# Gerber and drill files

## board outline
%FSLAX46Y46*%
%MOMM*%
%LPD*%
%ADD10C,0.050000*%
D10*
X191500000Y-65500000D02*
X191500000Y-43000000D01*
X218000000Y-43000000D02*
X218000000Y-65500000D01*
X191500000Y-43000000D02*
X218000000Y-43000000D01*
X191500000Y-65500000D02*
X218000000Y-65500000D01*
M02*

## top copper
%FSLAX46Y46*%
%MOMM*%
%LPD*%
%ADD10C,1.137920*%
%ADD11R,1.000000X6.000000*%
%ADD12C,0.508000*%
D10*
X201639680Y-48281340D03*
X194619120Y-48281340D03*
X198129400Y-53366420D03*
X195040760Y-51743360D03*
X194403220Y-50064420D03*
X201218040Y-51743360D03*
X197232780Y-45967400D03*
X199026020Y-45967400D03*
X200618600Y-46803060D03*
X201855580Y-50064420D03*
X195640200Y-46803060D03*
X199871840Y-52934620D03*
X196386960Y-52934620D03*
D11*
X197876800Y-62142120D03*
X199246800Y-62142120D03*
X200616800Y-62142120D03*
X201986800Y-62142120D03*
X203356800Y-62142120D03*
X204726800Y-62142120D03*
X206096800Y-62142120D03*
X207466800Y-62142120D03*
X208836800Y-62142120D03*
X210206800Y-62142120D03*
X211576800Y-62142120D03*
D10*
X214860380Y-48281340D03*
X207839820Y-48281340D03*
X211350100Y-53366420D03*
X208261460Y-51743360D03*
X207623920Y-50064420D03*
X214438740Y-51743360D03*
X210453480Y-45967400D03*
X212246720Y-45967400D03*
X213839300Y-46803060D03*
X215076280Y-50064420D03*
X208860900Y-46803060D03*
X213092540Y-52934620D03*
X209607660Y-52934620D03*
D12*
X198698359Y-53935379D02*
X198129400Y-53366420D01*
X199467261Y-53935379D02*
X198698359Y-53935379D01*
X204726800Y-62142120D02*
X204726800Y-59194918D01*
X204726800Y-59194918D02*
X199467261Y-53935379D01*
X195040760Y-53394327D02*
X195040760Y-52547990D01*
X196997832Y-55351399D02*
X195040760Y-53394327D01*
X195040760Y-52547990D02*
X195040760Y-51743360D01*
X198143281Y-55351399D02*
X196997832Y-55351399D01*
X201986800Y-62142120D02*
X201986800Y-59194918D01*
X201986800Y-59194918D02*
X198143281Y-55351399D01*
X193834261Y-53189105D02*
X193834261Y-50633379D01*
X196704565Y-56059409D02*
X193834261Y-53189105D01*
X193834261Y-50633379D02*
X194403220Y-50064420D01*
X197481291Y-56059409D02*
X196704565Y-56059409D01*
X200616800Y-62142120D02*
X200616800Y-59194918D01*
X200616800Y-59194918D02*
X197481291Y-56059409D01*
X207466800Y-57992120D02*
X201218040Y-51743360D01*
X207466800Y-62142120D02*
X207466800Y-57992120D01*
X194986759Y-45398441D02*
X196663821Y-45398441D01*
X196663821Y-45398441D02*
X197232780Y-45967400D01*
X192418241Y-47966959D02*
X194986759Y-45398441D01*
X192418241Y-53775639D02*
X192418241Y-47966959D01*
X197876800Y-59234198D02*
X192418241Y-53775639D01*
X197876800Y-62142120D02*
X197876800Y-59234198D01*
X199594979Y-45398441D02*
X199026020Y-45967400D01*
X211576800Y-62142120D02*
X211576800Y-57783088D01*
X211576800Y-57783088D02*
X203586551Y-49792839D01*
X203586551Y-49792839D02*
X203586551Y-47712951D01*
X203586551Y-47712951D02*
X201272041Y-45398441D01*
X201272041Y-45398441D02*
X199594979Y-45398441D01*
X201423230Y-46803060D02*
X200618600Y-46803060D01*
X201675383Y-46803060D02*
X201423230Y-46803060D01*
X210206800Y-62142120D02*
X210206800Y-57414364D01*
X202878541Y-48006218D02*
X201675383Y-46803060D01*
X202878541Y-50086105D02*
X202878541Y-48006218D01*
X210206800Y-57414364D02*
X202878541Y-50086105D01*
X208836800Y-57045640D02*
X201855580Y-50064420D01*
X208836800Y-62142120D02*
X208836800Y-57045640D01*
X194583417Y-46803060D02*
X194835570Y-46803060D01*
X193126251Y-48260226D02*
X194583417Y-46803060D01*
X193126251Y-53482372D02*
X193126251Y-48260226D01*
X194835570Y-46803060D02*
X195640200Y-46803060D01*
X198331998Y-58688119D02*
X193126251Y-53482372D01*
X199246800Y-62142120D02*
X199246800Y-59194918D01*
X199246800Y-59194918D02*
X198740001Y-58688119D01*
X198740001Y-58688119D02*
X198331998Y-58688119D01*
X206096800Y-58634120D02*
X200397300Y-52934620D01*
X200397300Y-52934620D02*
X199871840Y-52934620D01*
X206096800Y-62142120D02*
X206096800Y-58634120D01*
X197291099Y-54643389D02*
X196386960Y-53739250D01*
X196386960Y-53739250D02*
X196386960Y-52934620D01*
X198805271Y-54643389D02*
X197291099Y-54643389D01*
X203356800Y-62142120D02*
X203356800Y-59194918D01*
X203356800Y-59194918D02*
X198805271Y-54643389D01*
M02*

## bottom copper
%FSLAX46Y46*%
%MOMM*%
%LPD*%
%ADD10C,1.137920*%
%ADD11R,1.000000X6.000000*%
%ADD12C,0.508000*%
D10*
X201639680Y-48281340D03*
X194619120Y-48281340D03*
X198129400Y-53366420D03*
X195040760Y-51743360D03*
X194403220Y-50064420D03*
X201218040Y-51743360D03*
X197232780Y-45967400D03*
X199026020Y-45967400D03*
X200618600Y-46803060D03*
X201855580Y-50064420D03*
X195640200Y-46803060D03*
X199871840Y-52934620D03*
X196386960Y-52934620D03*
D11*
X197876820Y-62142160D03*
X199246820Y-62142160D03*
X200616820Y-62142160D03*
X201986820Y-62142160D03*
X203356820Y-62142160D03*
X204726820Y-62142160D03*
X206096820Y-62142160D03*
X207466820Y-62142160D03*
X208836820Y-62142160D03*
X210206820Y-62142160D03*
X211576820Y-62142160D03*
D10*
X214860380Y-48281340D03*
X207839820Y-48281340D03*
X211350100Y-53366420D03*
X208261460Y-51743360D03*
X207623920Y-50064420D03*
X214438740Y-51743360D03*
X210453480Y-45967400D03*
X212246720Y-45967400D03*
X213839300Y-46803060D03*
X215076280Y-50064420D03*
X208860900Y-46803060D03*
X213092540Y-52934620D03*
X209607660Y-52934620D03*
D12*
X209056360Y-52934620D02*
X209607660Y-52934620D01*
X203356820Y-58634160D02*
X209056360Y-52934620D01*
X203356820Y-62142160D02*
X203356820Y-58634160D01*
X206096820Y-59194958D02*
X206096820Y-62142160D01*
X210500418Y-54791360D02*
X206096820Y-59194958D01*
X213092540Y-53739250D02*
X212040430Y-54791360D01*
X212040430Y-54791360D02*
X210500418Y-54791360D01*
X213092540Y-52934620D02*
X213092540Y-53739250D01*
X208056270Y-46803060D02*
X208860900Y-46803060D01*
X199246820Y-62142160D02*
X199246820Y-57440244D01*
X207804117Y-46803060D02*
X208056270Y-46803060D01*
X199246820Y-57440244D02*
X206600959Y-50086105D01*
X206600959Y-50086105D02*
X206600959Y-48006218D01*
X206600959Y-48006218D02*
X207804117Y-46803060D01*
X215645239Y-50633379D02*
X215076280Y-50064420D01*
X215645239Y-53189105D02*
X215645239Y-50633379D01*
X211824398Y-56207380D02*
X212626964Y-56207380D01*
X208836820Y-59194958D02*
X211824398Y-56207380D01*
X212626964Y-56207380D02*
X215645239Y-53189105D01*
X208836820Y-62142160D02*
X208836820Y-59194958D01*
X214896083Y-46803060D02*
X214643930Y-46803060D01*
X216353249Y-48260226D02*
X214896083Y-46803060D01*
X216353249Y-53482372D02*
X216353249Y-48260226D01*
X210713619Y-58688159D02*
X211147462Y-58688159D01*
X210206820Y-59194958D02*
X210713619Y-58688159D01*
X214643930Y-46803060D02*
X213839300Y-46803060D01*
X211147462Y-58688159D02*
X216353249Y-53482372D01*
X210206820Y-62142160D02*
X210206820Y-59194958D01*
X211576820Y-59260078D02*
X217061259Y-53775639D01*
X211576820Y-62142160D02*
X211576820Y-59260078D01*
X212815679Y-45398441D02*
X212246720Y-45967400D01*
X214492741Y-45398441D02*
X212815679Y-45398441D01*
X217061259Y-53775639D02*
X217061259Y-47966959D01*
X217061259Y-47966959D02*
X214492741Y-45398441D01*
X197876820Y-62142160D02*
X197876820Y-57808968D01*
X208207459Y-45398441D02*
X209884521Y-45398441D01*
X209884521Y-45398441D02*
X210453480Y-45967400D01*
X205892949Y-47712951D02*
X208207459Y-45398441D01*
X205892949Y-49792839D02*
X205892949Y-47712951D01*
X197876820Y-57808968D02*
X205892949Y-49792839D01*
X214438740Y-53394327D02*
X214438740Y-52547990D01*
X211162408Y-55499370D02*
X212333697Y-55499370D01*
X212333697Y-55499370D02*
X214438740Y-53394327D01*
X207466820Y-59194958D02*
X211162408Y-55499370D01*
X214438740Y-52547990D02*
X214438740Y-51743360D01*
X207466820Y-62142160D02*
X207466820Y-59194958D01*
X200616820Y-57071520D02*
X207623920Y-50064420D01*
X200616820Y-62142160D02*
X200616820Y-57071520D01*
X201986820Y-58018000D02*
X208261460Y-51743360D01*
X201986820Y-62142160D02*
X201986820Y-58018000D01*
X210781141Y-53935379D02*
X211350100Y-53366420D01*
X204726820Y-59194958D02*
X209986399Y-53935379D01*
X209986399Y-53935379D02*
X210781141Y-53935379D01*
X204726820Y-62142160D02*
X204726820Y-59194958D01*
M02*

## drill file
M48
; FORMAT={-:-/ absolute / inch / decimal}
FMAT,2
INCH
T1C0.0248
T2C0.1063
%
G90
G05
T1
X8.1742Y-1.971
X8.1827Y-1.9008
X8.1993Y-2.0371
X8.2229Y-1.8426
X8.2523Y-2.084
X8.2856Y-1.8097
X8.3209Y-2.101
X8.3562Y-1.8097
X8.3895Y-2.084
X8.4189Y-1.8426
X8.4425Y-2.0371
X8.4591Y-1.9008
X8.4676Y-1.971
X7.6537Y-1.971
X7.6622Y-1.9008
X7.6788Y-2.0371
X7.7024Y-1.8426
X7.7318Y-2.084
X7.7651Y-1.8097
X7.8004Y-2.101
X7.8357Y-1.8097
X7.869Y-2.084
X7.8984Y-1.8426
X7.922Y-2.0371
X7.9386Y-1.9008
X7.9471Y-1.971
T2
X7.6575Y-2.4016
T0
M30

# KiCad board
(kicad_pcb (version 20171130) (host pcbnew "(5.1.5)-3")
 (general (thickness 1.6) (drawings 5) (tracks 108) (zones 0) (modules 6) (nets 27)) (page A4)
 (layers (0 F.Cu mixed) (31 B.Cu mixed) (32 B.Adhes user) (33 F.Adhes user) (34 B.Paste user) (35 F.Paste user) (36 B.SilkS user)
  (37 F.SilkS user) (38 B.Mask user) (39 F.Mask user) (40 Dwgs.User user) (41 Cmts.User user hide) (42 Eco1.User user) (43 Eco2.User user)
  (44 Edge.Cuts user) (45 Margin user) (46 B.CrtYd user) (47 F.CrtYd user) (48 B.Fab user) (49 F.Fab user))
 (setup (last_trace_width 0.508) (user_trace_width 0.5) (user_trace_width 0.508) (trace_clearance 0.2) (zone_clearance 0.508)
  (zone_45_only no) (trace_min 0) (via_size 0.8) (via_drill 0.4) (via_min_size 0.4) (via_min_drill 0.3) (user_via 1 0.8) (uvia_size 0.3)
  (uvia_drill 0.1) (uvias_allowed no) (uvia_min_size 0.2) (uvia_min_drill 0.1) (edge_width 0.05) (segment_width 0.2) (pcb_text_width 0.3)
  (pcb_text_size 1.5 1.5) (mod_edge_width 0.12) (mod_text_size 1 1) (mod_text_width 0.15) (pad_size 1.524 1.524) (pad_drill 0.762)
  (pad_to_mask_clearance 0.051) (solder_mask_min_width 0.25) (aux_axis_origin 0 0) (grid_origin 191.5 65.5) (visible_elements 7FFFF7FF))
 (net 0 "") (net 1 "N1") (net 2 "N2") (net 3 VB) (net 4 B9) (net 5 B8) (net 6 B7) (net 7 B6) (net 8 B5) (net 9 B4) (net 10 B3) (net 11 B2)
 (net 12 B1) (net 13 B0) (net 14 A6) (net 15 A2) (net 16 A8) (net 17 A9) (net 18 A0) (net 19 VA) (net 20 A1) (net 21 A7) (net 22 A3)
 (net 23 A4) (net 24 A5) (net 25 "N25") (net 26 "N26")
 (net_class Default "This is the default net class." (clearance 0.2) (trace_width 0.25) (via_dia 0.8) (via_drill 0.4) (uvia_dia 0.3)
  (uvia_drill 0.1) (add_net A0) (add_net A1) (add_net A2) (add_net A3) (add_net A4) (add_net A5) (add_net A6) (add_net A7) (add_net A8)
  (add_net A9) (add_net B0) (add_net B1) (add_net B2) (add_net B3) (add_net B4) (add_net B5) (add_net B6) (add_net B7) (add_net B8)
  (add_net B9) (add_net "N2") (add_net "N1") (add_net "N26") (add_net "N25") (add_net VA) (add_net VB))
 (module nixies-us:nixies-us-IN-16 (layer F.Cu) (at 198.1294 49.6123)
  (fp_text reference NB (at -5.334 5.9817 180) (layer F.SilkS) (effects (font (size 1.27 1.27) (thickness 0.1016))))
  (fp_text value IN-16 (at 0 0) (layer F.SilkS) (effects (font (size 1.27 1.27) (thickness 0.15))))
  (pad RHDP thru_hole circle (at 3.51028 -1.33096) (size 1.13792 1.13792) (drill 0.62992) (layers *.Cu *.Mask) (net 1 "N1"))
  (pad LHDP thru_hole circle (at -3.51028 -1.33096) (size 1.13792 1.13792) (drill 0.62992) (layers *.Cu *.Mask) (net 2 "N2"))
  (pad A thru_hole circle (at 0 3.75412) (size 1.13792 1.13792) (drill 0.62992) (layers *.Cu *.Mask) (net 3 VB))
  (pad 9 thru_hole circle (at -3.08864 2.13106) (size 1.13792 1.13792) (drill 0.62992) (layers *.Cu *.Mask) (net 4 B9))
  (pad 8 thru_hole circle (at -3.72618 0.45212) (size 1.13792 1.13792) (drill 0.62992) (layers *.Cu *.Mask) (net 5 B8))
  (pad 7 thru_hole circle (at 3.08864 2.13106) (size 1.13792 1.13792) (drill 0.62992) (layers *.Cu *.Mask) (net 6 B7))
  (pad 6 thru_hole circle (at -0.89662 -3.6449) (size 1.13792 1.13792) (drill 0.62992) (layers *.Cu *.Mask) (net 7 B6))
  (pad 5 thru_hole circle (at 0.89662 -3.6449) (size 1.13792 1.13792) (drill 0.62992) (layers *.Cu *.Mask) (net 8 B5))
  (pad 4 thru_hole circle (at 2.4892 -2.80924) (size 1.13792 1.13792) (drill 0.62992) (layers *.Cu *.Mask) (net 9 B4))
  (pad 3 thru_hole circle (at 3.72618 0.45212) (size 1.13792 1.13792) (drill 0.62992) (layers *.Cu *.Mask) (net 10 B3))
  (pad 2 thru_hole circle (at -2.4892 -2.80924) (size 1.13792 1.13792) (drill 0.62992) (layers *.Cu *.Mask) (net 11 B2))
  (pad 1 thru_hole circle (at 1.74244 3.32232) (size 1.13792 1.13792) (drill 0.62992) (layers *.Cu *.Mask) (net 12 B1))
  (pad 0 thru_hole circle (at -1.74244 3.32232) (size 1.13792 1.13792) (drill 0.62992) (layers *.Cu *.Mask) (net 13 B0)))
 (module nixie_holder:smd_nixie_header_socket (layer B.Cu) (at 197.87682 62.14216)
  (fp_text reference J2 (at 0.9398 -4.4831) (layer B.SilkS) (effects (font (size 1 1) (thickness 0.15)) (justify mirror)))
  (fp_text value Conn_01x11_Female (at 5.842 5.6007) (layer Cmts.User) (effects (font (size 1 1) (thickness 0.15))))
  (pad 1 smd rect (at 0 0) (size 1 6) (layers B.Cu B.Paste B.Mask) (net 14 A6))
  (pad 2 smd rect (at 1.37 0) (size 1 6) (layers B.Cu B.Paste B.Mask) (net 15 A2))
  (pad 3 smd rect (at 2.74 0) (size 1 6) (layers B.Cu B.Paste B.Mask) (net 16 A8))
  (pad 4 smd rect (at 4.11 0) (size 1 6) (layers B.Cu B.Paste B.Mask) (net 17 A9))
  (pad 5 smd rect (at 5.48 0) (size 1 6) (layers B.Cu B.Paste B.Mask) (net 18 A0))
  (pad 6 smd rect (at 6.85 0) (size 1 6) (layers B.Cu B.Paste B.Mask) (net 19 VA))
  (pad 7 smd rect (at 8.22 0) (size 1 6) (layers B.Cu B.Paste B.Mask) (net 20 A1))
  (pad 8 smd rect (at 9.59 0) (size 1 6) (layers B.Cu B.Paste B.Mask) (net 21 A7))
  (pad 9 smd rect (at 10.96 0) (size 1 6) (layers B.Cu B.Paste B.Mask) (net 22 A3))
  (pad 10 smd rect (at 12.33 0) (size 1 6) (layers B.Cu B.Paste B.Mask) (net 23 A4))
  (pad 11 smd rect (at 13.7 0) (size 1 6) (layers B.Cu B.Paste B.Mask) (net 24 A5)))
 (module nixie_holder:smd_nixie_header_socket (layer F.Cu) (at 197.8768 62.14212)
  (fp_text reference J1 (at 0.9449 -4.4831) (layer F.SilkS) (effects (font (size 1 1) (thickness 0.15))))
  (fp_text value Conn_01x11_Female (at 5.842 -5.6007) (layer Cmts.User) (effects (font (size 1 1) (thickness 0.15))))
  (pad 1 smd rect (at 0 0) (size 1 6) (layers F.Cu F.Paste F.Mask) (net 7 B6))
  (pad 2 smd rect (at 1.37 0) (size 1 6) (layers F.Cu F.Paste F.Mask) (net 11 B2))
  (pad 3 smd rect (at 2.74 0) (size 1 6) (layers F.Cu F.Paste F.Mask) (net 5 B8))
  (pad 4 smd rect (at 4.11 0) (size 1 6) (layers F.Cu F.Paste F.Mask) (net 4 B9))
  (pad 5 smd rect (at 5.48 0) (size 1 6) (layers F.Cu F.Paste F.Mask) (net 13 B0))
  (pad 6 smd rect (at 6.85 0) (size 1 6) (layers F.Cu F.Paste F.Mask) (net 3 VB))
  (pad 7 smd rect (at 8.22 0) (size 1 6) (layers F.Cu F.Paste F.Mask) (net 12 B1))
  (pad 8 smd rect (at 9.59 0) (size 1 6) (layers F.Cu F.Paste F.Mask) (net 6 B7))
  (pad 9 smd rect (at 10.96 0) (size 1 6) (layers F.Cu F.Paste F.Mask) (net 10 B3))
  (pad 10 smd rect (at 12.33 0) (size 1 6) (layers F.Cu F.Paste F.Mask) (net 9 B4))
  (pad 11 smd rect (at 13.7 0) (size 1 6) (layers F.Cu F.Paste F.Mask) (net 8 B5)))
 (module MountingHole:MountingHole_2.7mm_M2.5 (layer F.Cu) (at 194.5 61)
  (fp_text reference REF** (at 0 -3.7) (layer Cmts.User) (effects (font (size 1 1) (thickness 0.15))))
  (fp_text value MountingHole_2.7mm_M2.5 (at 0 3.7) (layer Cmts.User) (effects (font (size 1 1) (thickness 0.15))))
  (pad 1 np_thru_hole circle (at 0 0) (size 2.7 2.7) (drill 2.7) (layers *.Cu *.Mask)))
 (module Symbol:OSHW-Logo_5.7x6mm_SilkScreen (layer F.Cu) (at 204.708 55.81244)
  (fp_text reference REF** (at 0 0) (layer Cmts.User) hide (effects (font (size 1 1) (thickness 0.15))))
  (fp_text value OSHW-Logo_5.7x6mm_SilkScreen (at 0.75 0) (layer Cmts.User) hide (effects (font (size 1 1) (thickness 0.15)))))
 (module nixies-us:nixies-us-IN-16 (layer F.Cu) (at 211.3501 49.6123)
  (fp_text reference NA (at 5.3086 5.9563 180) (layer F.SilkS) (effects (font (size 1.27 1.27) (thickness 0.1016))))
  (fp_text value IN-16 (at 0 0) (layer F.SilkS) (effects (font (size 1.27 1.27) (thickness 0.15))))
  (pad RHDP thru_hole circle (at 3.51028 -1.33096) (size 1.13792 1.13792) (drill 0.62992) (layers *.Cu *.Mask) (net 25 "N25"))
  (pad LHDP thru_hole circle (at -3.51028 -1.33096) (size 1.13792 1.13792) (drill 0.62992) (layers *.Cu *.Mask) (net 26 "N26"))
  (pad A thru_hole circle (at 0 3.75412) (size 1.13792 1.13792) (drill 0.62992) (layers *.Cu *.Mask) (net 19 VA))
  (pad 9 thru_hole circle (at -3.08864 2.13106) (size 1.13792 1.13792) (drill 0.62992) (layers *.Cu *.Mask) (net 17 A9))
  (pad 8 thru_hole circle (at -3.72618 0.45212) (size 1.13792 1.13792) (drill 0.62992) (layers *.Cu *.Mask) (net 16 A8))
  (pad 7 thru_hole circle (at 3.08864 2.13106) (size 1.13792 1.13792) (drill 0.62992) (layers *.Cu *.Mask) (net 21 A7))
  (pad 6 thru_hole circle (at -0.89662 -3.6449) (size 1.13792 1.13792) (drill 0.62992) (layers *.Cu *.Mask) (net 14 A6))
  (pad 5 thru_hole circle (at 0.89662 -3.6449) (size 1.13792 1.13792) (drill 0.62992) (layers *.Cu *.Mask) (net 24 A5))
  (pad 4 thru_hole circle (at 2.4892 -2.80924) (size 1.13792 1.13792) (drill 0.62992) (layers *.Cu *.Mask) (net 23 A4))
  (pad 3 thru_hole circle (at 3.72618 0.45212) (size 1.13792 1.13792) (drill 0.62992) (layers *.Cu *.Mask) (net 22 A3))
  (pad 2 thru_hole circle (at -2.4892 -2.80924) (size 1.13792 1.13792) (drill 0.62992) (layers *.Cu *.Mask) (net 15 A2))
  (pad 1 thru_hole circle (at 1.74244 3.32232) (size 1.13792 1.13792) (drill 0.62992) (layers *.Cu *.Mask) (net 20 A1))
  (pad 0 thru_hole circle (at -1.74244 3.32232) (size 1.13792 1.13792) (drill 0.62992) (layers *.Cu *.Mask) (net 18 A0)))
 (gr_line (start 191.5 65.5) (end 191.5 43) (layer Edge.Cuts) (width 0.05))
 (gr_line (start 218 43) (end 218 65.5) (layer Edge.Cuts) (width 0.05))
 (gr_line (start 191.5 43) (end 218 43) (layer Edge.Cuts) (width 0.05))
 (gr_line (start 191.5 65.5) (end 218 65.5) (layer Edge.Cuts) (width 0.05))
 (segment (start 198.698359 53.935379) (end 198.1294 53.36642) (width 0.508) (layer F.Cu) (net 3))
 (segment (start 199.467261 53.935379) (end 198.698359 53.935379) (width 0.508) (layer F.Cu) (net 3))
 (segment (start 204.7268 62.14212) (end 204.7268 59.194918) (width 0.508) (layer F.Cu) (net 3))
 (segment (start 204.7268 59.194918) (end 199.467261 53.935379) (width 0.508) (layer F.Cu) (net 3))
 (segment (start 195.04076 53.394327) (end 195.04076 52.54799) (width 0.508) (layer F.Cu) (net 4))
 (segment (start 196.997832 55.351399) (end 195.04076 53.394327) (width 0.508) (layer F.Cu) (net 4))
 (segment (start 195.04076 52.54799) (end 195.04076 51.74336) (width 0.508) (layer F.Cu) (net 4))
 (segment (start 198.143281 55.351399) (end 196.997832 55.351399) (width 0.508) (layer F.Cu) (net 4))
 (segment (start 201.9868 62.14212) (end 201.9868 59.194918) (width 0.508) (layer F.Cu) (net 4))
 (segment (start 201.9868 59.194918) (end 198.143281 55.351399) (width 0.508) (layer F.Cu) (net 4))
 (segment (start 193.834261 53.189105) (end 193.834261 50.633379) (width 0.508) (layer F.Cu) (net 5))
 (segment (start 196.704565 56.059409) (end 193.834261 53.189105) (width 0.508) (layer F.Cu) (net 5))
 (segment (start 193.834261 50.633379) (end 194.40322 50.06442) (width 0.508) (layer F.Cu) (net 5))
 (segment (start 197.481291 56.059409) (end 196.704565 56.059409) (width 0.508) (layer F.Cu) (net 5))
 (segment (start 200.6168 62.14212) (end 200.6168 59.194918) (width 0.508) (layer F.Cu) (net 5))
 (segment (start 200.6168 59.194918) (end 197.481291 56.059409) (width 0.508) (layer F.Cu) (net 5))
 (segment (start 207.4668 57.99212) (end 201.21804 51.74336) (width 0.508) (layer F.Cu) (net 6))
 (segment (start 207.4668 62.14212) (end 207.4668 57.99212) (width 0.508) (layer F.Cu) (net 6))
 (segment (start 194.986759 45.398441) (end 196.663821 45.398441) (width 0.508) (layer F.Cu) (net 7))
 (segment (start 196.663821 45.398441) (end 197.23278 45.9674) (width 0.508) (layer F.Cu) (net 7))
 (segment (start 192.418241 47.966959) (end 194.986759 45.398441) (width 0.508) (layer F.Cu) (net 7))
 (segment (start 192.418241 53.775639) (end 192.418241 47.966959) (width 0.508) (layer F.Cu) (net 7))
 (segment (start 197.8768 59.234198) (end 192.418241 53.775639) (width 0.508) (layer F.Cu) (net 7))
 (segment (start 197.8768 62.14212) (end 197.8768 59.234198) (width 0.508) (layer F.Cu) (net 7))
 (segment (start 199.594979 45.398441) (end 199.02602 45.9674) (width 0.508) (layer F.Cu) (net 8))
 (segment (start 211.5768 62.14212) (end 211.5768 57.783088) (width 0.508) (layer F.Cu) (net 8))
 (segment (start 211.5768 57.783088) (end 203.586551 49.792839) (width 0.508) (layer F.Cu) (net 8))
 (segment (start 203.586551 49.792839) (end 203.586551 47.712951) (width 0.508) (layer F.Cu) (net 8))
 (segment (start 203.586551 47.712951) (end 201.272041 45.398441) (width 0.508) (layer F.Cu) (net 8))
 (segment (start 201.272041 45.398441) (end 199.594979 45.398441) (width 0.508) (layer F.Cu) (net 8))
 (segment (start 201.42323 46.80306) (end 200.6186 46.80306) (width 0.508) (layer F.Cu) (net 9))
 (segment (start 201.675383 46.80306) (end 201.42323 46.80306) (width 0.508) (layer F.Cu) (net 9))
 (segment (start 210.2068 62.14212) (end 210.2068 57.414364) (width 0.508) (layer F.Cu) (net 9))
 (segment (start 202.878541 48.006218) (end 201.675383 46.80306) (width 0.508) (layer F.Cu) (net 9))
 (segment (start 202.878541 50.086105) (end 202.878541 48.006218) (width 0.508) (layer F.Cu) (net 9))
 (segment (start 210.2068 57.414364) (end 202.878541 50.086105) (width 0.508) (layer F.Cu) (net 9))
 (segment (start 208.8368 57.04564) (end 201.85558 50.06442) (width 0.508) (layer F.Cu) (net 10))
 (segment (start 208.8368 62.14212) (end 208.8368 57.04564) (width 0.508) (layer F.Cu) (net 10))
 (segment (start 194.583417 46.80306) (end 194.83557 46.80306) (width 0.508) (layer F.Cu) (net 11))
 (segment (start 193.126251 48.260226) (end 194.583417 46.80306) (width 0.508) (layer F.Cu) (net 11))
 (segment (start 193.126251 53.482372) (end 193.126251 48.260226) (width 0.508) (layer F.Cu) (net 11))
 (segment (start 194.83557 46.80306) (end 195.6402 46.80306) (width 0.508) (layer F.Cu) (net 11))
 (segment (start 198.331998 58.688119) (end 193.126251 53.482372) (width 0.508) (layer F.Cu) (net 11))
 (segment (start 199.2468 62.14212) (end 199.2468 59.194918) (width 0.508) (layer F.Cu) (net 11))
 (segment (start 199.2468 59.194918) (end 198.740001 58.688119) (width 0.508) (layer F.Cu) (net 11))
 (segment (start 198.740001 58.688119) (end 198.331998 58.688119) (width 0.508) (layer F.Cu) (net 11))
 (segment (start 206.0968 58.63412) (end 200.3973 52.93462) (width 0.508) (layer F.Cu) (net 12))
 (segment (start 200.3973 52.93462) (end 199.87184 52.93462) (width 0.508) (layer F.Cu) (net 12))
 (segment (start 206.0968 62.14212) (end 206.0968 58.63412) (width 0.508) (layer F.Cu) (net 12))
 (segment (start 197.291099 54.643389) (end 196.38696 53.73925) (width 0.508) (layer F.Cu) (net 13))
 (segment (start 196.38696 53.73925) (end 196.38696 52.93462) (width 0.508) (layer F.Cu) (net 13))
 (segment (start 198.805271 54.643389) (end 197.291099 54.643389) (width 0.508) (layer F.Cu) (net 13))
 (segment (start 203.3568 62.14212) (end 203.3568 59.194918) (width 0.508) (layer F.Cu) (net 13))
 (segment (start 203.3568 59.194918) (end 198.805271 54.643389) (width 0.508) (layer F.Cu) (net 13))
 (segment (start 209.05636 52.93462) (end 209.60766 52.93462) (width 0.508) (layer B.Cu) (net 18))
 (segment (start 203.35682 58.63416) (end 209.05636 52.93462) (width 0.508) (layer B.Cu) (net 18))
 (segment (start 203.35682 62.14216) (end 203.35682 58.63416) (width 0.508) (layer B.Cu) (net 18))
 (segment (start 206.09682 59.194958) (end 206.09682 62.14216) (width 0.508) (layer B.Cu) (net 20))
 (segment (start 210.500418 54.79136) (end 206.09682 59.194958) (width 0.508) (layer B.Cu) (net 20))
 (segment (start 213.09254 53.73925) (end 212.04043 54.79136) (width 0.508) (layer B.Cu) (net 20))
 (segment (start 212.04043 54.79136) (end 210.500418 54.79136) (width 0.508) (layer B.Cu) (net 20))
 (segment (start 213.09254 52.93462) (end 213.09254 53.73925) (width 0.508) (layer B.Cu) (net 20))
 (segment (start 208.05627 46.80306) (end 208.8609 46.80306) (width 0.508) (layer B.Cu) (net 15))
 (segment (start 199.24682 62.14216) (end 199.24682 57.440244) (width 0.508) (layer B.Cu) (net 15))
 (segment (start 207.804117 46.80306) (end 208.05627 46.80306) (width 0.508) (layer B.Cu) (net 15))
 (segment (start 199.24682 57.440244) (end 206.600959 50.086105) (width 0.508) (layer B.Cu) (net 15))
 (segment (start 206.600959 50.086105) (end 206.600959 48.006218) (width 0.508) (layer B.Cu) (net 15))
 (segment (start 206.600959 48.006218) (end 207.804117 46.80306) (width 0.508) (layer B.Cu) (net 15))
 (segment (start 215.645239 50.633379) (end 215.07628 50.06442) (width 0.508) (layer B.Cu) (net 22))
 (segment (start 215.645239 53.189105) (end 215.645239 50.633379) (width 0.508) (layer B.Cu) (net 22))
 (segment (start 211.824398 56.20738) (end 212.626964 56.20738) (width 0.508) (layer B.Cu) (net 22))
 (segment (start 208.83682 59.194958) (end 211.824398 56.20738) (width 0.508) (layer B.Cu) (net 22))
 (segment (start 212.626964 56.20738) (end 215.645239 53.189105) (width 0.508) (layer B.Cu) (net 22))
 (segment (start 208.83682 62.14216) (end 208.83682 59.194958) (width 0.508) (layer B.Cu) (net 22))
 (segment (start 214.896083 46.80306) (end 214.64393 46.80306) (width 0.508) (layer B.Cu) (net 23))
 (segment (start 216.353249 48.260226) (end 214.896083 46.80306) (width 0.508) (layer B.Cu) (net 23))
 (segment (start 216.353249 53.482372) (end 216.353249 48.260226) (width 0.508) (layer B.Cu) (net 23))
 (segment (start 210.713619 58.688159) (end 211.147462 58.688159) (width 0.508) (layer B.Cu) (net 23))
 (segment (start 210.20682 59.194958) (end 210.713619 58.688159) (width 0.508) (layer B.Cu) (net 23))
 (segment (start 214.64393 46.80306) (end 213.8393 46.80306) (width 0.508) (layer B.Cu) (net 23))
 (segment (start 211.147462 58.688159) (end 216.353249 53.482372) (width 0.508) (layer B.Cu) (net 23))
 (segment (start 210.20682 62.14216) (end 210.20682 59.194958) (width 0.508) (layer B.Cu) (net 23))
 (segment (start 211.57682 59.260078) (end 217.061259 53.775639) (width 0.508) (layer B.Cu) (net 24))
 (segment (start 211.57682 62.14216) (end 211.57682 59.260078) (width 0.508) (layer B.Cu) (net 24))
 (segment (start 212.815679 45.398441) (end 212.24672 45.9674) (width 0.508) (layer B.Cu) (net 24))
 (segment (start 214.492741 45.398441) (end 212.815679 45.398441) (width 0.508) (layer B.Cu) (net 24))
 (segment (start 217.061259 53.775639) (end 217.061259 47.966959) (width 0.508) (layer B.Cu) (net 24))
 (segment (start 217.061259 47.966959) (end 214.492741 45.398441) (width 0.508) (layer B.Cu) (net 24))
 (segment (start 197.87682 62.14216) (end 197.87682 57.808968) (width 0.508) (layer B.Cu) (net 14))
 (segment (start 208.207459 45.398441) (end 209.884521 45.398441) (width 0.508) (layer B.Cu) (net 14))
 (segment (start 209.884521 45.398441) (end 210.45348 45.9674) (width 0.508) (layer B.Cu) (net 14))
 (segment (start 205.892949 47.712951) (end 208.207459 45.398441) (width 0.508) (layer B.Cu) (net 14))
 (segment (start 205.892949 49.792839) (end 205.892949 47.712951) (width 0.508) (layer B.Cu) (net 14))
 (segment (start 197.87682 57.808968) (end 205.892949 49.792839) (width 0.508) (layer B.Cu) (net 14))
 (segment (start 214.43874 53.394327) (end 214.43874 52.54799) (width 0.508) (layer B.Cu) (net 21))
 (segment (start 211.162408 55.49937) (end 212.333697 55.49937) (width 0.508) (layer B.Cu) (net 21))
 (segment (start 212.333697 55.49937) (end 214.43874 53.394327) (width 0.508) (layer B.Cu) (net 21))
 (segment (start 207.46682 59.194958) (end 211.162408 55.49937) (width 0.508) (layer B.Cu) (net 21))
 (segment (start 214.43874 52.54799) (end 214.43874 51.74336) (width 0.508) (layer B.Cu) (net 21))
 (segment (start 207.46682 62.14216) (end 207.46682 59.194958) (width 0.508) (layer B.Cu) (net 21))
 (segment (start 200.61682 57.07152) (end 207.62392 50.06442) (width 0.508) (layer B.Cu) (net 16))
 (segment (start 200.61682 62.14216) (end 200.61682 57.07152) (width 0.508) (layer B.Cu) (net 16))
 (segment (start 201.98682 58.018) (end 208.26146 51.74336) (width 0.508) (layer B.Cu) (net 17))
 (segment (start 201.98682 62.14216) (end 201.98682 58.018) (width 0.508) (layer B.Cu) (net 17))
 (segment (start 210.781141 53.935379) (end 211.3501 53.36642) (width 0.508) (layer B.Cu) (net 19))
 (segment (start 204.72682 59.194958) (end 209.986399 53.935379) (width 0.508) (layer B.Cu) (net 19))
 (segment (start 209.986399 53.935379) (end 210.781141 53.935379) (width 0.508) (layer B.Cu) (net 19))
 (segment (start 204.72682 62.14216) (end 204.72682 59.194958) (width 0.508) (layer B.Cu) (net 19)))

